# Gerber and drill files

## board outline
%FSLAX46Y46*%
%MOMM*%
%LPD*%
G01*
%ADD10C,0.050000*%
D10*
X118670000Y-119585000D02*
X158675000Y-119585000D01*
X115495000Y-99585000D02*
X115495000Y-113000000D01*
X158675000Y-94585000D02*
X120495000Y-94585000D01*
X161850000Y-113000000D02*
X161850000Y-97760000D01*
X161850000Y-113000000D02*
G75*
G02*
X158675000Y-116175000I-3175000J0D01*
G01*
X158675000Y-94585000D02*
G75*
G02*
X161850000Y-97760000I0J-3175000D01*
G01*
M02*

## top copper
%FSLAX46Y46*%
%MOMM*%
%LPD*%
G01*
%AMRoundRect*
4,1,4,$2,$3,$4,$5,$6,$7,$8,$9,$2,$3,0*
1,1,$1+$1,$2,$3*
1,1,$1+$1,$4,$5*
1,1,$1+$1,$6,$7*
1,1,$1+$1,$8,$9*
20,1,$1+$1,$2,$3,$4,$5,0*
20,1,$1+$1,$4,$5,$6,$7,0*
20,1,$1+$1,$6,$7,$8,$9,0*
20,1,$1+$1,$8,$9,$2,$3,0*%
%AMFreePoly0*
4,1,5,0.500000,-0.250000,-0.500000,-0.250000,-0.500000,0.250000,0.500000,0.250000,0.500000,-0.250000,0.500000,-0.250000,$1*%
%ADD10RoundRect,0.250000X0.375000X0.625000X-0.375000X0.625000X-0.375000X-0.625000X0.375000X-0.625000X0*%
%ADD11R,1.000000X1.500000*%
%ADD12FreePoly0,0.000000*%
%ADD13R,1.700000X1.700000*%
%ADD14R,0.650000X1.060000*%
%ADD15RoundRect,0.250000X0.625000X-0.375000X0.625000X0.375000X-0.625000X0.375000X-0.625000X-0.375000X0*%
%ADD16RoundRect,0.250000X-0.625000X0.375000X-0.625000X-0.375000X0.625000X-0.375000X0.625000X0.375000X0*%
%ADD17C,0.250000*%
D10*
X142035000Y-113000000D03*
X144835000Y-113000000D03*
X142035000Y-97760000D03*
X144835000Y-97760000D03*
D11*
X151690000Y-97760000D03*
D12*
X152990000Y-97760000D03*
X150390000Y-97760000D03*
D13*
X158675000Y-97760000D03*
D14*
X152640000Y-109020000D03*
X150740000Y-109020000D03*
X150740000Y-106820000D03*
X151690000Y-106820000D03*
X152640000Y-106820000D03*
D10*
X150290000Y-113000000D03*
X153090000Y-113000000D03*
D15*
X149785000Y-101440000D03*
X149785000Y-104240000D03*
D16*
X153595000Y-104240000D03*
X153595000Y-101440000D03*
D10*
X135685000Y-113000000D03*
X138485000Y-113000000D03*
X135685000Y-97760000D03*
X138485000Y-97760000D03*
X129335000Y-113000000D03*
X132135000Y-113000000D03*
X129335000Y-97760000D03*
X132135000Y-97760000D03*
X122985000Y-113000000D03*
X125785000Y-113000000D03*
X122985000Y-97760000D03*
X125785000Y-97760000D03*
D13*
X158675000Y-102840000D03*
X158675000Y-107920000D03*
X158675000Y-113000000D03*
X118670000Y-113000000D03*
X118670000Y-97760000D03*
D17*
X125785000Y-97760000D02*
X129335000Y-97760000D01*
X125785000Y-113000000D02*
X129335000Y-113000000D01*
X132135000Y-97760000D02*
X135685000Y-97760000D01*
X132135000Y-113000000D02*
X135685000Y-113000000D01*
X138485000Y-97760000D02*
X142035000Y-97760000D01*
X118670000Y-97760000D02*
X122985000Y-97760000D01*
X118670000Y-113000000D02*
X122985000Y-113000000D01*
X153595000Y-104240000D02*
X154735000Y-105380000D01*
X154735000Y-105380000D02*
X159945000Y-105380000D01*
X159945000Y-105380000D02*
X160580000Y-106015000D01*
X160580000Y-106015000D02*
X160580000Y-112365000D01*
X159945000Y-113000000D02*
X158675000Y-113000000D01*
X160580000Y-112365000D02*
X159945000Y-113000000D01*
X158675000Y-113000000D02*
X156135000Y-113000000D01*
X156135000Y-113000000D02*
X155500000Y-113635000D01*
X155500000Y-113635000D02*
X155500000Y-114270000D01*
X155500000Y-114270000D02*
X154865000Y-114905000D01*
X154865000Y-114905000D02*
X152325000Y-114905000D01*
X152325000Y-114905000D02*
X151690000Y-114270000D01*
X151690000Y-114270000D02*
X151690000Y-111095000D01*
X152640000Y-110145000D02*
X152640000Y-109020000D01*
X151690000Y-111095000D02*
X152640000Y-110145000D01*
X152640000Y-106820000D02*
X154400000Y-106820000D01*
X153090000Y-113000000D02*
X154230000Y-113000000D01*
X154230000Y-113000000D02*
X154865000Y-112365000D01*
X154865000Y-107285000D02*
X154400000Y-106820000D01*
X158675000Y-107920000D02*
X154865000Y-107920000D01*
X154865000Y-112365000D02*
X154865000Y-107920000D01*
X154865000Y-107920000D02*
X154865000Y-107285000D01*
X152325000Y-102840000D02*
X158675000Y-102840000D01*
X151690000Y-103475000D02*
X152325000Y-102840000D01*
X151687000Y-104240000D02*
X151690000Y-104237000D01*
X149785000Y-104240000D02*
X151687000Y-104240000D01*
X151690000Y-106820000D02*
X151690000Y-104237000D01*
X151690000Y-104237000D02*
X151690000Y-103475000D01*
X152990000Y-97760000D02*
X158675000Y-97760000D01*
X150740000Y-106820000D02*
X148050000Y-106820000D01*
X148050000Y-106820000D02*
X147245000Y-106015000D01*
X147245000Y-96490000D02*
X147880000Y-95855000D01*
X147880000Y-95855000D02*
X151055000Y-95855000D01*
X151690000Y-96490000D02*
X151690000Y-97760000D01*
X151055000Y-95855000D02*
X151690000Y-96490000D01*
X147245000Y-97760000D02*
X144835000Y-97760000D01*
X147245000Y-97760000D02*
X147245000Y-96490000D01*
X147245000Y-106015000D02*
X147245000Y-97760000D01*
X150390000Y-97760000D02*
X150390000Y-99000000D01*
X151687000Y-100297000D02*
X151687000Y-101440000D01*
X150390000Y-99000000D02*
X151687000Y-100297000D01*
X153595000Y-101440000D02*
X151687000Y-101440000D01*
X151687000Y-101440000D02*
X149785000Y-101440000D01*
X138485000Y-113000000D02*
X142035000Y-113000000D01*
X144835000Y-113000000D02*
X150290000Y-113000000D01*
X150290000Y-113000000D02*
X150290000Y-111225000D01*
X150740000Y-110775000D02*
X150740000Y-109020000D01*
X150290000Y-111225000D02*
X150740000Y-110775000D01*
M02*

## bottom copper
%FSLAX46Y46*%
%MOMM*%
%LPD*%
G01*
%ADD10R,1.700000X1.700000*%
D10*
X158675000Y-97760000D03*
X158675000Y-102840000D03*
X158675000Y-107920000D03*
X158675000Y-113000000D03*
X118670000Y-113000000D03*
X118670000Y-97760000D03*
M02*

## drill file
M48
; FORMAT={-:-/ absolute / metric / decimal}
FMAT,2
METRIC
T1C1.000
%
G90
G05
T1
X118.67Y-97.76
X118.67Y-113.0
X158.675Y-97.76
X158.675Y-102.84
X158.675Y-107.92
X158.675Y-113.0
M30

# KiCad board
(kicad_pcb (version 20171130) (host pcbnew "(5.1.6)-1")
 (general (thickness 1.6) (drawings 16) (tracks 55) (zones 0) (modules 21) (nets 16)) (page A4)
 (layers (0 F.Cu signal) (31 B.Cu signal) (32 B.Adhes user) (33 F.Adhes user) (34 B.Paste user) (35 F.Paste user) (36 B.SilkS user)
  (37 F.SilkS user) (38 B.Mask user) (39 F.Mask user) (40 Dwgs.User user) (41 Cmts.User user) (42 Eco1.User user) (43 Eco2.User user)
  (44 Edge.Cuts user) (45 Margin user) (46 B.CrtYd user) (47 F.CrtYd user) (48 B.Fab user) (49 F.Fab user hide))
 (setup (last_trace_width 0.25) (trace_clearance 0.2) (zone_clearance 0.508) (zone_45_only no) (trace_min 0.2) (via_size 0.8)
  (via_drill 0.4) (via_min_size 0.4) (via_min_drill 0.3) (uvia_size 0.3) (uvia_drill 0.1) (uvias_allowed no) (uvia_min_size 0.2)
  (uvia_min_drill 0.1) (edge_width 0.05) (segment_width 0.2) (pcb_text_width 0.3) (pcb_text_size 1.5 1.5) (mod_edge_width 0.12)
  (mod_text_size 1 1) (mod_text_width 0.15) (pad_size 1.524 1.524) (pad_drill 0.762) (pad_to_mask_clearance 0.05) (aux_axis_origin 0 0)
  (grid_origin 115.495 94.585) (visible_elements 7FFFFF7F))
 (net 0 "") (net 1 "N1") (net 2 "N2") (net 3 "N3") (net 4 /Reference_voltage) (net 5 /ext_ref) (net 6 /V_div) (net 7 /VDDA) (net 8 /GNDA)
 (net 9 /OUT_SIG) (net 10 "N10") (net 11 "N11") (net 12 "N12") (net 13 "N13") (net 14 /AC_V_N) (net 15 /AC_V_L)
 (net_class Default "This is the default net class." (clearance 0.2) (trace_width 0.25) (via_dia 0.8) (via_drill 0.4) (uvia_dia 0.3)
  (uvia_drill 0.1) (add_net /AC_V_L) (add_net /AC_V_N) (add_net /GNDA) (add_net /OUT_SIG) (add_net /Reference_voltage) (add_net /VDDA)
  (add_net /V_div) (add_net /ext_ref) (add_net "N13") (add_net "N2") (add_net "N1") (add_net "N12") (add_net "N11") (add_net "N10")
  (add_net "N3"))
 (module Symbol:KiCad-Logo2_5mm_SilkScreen (layer F.Cu) (at 129.465 105.38)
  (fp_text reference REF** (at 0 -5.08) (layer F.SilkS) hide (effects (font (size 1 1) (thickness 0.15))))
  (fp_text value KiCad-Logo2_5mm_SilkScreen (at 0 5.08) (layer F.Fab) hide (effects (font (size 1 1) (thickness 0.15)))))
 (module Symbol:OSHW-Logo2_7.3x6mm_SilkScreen (layer F.Cu) (at 142.165 105.38)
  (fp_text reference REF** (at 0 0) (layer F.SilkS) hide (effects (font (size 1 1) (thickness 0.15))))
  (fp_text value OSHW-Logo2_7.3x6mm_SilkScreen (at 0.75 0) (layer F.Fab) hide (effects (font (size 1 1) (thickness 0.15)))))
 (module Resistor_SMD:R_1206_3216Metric (layer F.Cu) (at 143.435 113 180)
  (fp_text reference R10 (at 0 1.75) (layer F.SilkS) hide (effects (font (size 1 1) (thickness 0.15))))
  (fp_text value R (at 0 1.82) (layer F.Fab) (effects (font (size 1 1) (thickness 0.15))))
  (pad 2 smd roundrect (at 1.4 0 180) (size 1.25 1.75) (layers F.Cu F.Paste F.Mask) (roundrect_rratio 0.2) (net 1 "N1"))
  (pad 1 smd roundrect (at -1.4 0 180) (size 1.25 1.75) (layers F.Cu F.Paste F.Mask) (roundrect_rratio 0.2) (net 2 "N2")))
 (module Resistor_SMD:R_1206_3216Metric (layer F.Cu) (at 143.435 97.76 180)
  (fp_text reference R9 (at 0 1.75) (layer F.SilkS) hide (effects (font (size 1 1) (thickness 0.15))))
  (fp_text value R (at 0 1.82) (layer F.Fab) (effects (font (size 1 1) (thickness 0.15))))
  (pad 2 smd roundrect (at 1.4 0 180) (size 1.25 1.75) (layers F.Cu F.Paste F.Mask) (roundrect_rratio 0.2) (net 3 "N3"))
  (pad 1 smd roundrect (at -1.4 0 180) (size 1.25 1.75) (layers F.Cu F.Paste F.Mask) (roundrect_rratio 0.2) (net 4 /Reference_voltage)))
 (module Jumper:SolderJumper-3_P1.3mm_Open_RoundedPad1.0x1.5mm (layer F.Cu) (at 151.69 97.76)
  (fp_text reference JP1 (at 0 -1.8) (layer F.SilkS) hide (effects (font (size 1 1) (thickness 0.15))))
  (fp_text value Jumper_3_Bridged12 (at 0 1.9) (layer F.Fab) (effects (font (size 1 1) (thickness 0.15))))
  (pad 2 smd rect (at 0 0) (size 1 1.5) (layers F.Cu F.Mask) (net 4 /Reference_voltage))
  (pad 3 smd custom (at 1.3 0) (size 1 0.5) (layers F.Cu F.Mask) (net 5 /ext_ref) (zone_connect 2)
   (options (clearance outline) (anchor rect)) (primitives))
  (pad 1 smd custom (at -1.3 0) (size 1 0.5) (layers F.Cu F.Mask) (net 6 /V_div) (zone_connect 2)
   (options (clearance outline) (anchor rect)) (primitives)))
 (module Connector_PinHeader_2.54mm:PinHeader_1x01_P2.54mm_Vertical (layer F.Cu) (at 158.675 97.76)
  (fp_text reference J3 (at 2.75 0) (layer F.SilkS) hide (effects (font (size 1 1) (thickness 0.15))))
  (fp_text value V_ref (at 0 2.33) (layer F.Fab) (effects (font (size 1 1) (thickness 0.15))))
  (pad 1 thru_hole rect (at 0 0) (size 1.7 1.7) (drill 1) (layers *.Cu *.Mask) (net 5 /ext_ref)))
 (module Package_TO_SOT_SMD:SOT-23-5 (layer F.Cu) (at 151.69 107.92 270)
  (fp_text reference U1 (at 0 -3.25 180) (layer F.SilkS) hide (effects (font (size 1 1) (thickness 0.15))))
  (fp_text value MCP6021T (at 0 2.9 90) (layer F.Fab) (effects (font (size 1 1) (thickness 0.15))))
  (pad 5 smd rect (at 1.1 -0.95 270) (size 1.06 0.65) (layers F.Cu F.Paste F.Mask) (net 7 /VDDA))
  (pad 4 smd rect (at 1.1 0.95 270) (size 1.06 0.65) (layers F.Cu F.Paste F.Mask) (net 2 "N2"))
  (pad 3 smd rect (at -1.1 0.95 270) (size 1.06 0.65) (layers F.Cu F.Paste F.Mask) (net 4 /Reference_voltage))
  (pad 2 smd rect (at -1.1 0 270) (size 1.06 0.65) (layers F.Cu F.Paste F.Mask) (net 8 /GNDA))
  (pad 1 smd rect (at -1.1 -0.95 270) (size 1.06 0.65) (layers F.Cu F.Paste F.Mask) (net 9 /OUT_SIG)))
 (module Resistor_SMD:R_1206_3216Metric (layer F.Cu) (at 151.69 113 180)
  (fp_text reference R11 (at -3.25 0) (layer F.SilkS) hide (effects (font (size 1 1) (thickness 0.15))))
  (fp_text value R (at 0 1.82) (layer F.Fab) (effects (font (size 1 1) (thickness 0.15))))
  (pad 2 smd roundrect (at 1.4 0 180) (size 1.25 1.75) (layers F.Cu F.Paste F.Mask) (roundrect_rratio 0.2) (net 2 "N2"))
  (pad 1 smd roundrect (at -1.4 0 180) (size 1.25 1.75) (layers F.Cu F.Paste F.Mask) (roundrect_rratio 0.2) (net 9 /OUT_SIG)))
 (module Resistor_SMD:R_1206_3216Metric (layer F.Cu) (at 149.785 102.84 90)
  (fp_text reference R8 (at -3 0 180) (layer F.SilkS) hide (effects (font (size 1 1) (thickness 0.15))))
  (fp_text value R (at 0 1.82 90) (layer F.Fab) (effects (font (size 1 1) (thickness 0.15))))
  (pad 2 smd roundrect (at 1.4 0 90) (size 1.25 1.75) (layers F.Cu F.Paste F.Mask) (roundrect_rratio 0.2) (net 6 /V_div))
  (pad 1 smd roundrect (at -1.4 0 90) (size 1.25 1.75) (layers F.Cu F.Paste F.Mask) (roundrect_rratio 0.2) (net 8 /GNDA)))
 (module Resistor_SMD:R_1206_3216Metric (layer F.Cu) (at 153.595 102.84 270)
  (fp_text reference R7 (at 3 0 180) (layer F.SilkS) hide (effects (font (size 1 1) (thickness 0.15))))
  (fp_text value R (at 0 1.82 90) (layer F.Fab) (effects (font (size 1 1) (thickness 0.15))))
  (pad 2 smd roundrect (at 1.4 0 270) (size 1.25 1.75) (layers F.Cu F.Paste F.Mask) (roundrect_rratio 0.2) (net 7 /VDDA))
  (pad 1 smd roundrect (at -1.4 0 270) (size 1.25 1.75) (layers F.Cu F.Paste F.Mask) (roundrect_rratio 0.2) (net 6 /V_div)))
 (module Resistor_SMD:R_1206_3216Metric (layer F.Cu) (at 137.085 113 180)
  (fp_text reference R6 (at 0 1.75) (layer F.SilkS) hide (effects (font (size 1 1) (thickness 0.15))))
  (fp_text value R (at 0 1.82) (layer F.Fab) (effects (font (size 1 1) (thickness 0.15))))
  (pad 2 smd roundrect (at 1.4 0 180) (size 1.25 1.75) (layers F.Cu F.Paste F.Mask) (roundrect_rratio 0.2) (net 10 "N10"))
  (pad 1 smd roundrect (at -1.4 0 180) (size 1.25 1.75) (layers F.Cu F.Paste F.Mask) (roundrect_rratio 0.2) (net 1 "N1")))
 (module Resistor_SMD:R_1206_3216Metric (layer F.Cu) (at 137.085 97.76 180)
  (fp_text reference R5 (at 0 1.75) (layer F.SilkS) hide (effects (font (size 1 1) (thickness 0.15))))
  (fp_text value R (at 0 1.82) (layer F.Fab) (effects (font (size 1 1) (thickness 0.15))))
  (pad 2 smd roundrect (at 1.4 0 180) (size 1.25 1.75) (layers F.Cu F.Paste F.Mask) (roundrect_rratio 0.2) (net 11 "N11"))
  (pad 1 smd roundrect (at -1.4 0 180) (size 1.25 1.75) (layers F.Cu F.Paste F.Mask) (roundrect_rratio 0.2) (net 3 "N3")))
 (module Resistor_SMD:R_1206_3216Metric (layer F.Cu) (at 130.735 113 180)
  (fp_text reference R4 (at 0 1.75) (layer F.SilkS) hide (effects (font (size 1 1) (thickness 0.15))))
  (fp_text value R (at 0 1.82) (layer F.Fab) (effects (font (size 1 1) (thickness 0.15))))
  (pad 2 smd roundrect (at 1.4 0 180) (size 1.25 1.75) (layers F.Cu F.Paste F.Mask) (roundrect_rratio 0.2) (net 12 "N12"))
  (pad 1 smd roundrect (at -1.4 0 180) (size 1.25 1.75) (layers F.Cu F.Paste F.Mask) (roundrect_rratio 0.2) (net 10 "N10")))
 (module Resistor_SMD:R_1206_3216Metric (layer F.Cu) (at 130.735 97.76 180)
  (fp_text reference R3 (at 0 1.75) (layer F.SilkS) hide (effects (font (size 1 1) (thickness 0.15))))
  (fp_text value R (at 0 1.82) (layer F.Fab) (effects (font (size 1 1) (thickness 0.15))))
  (pad 2 smd roundrect (at 1.4 0 180) (size 1.25 1.75) (layers F.Cu F.Paste F.Mask) (roundrect_rratio 0.2) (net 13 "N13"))
  (pad 1 smd roundrect (at -1.4 0 180) (size 1.25 1.75) (layers F.Cu F.Paste F.Mask) (roundrect_rratio 0.2) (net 11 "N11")))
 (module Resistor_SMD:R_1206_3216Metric (layer F.Cu) (at 124.385 113 180)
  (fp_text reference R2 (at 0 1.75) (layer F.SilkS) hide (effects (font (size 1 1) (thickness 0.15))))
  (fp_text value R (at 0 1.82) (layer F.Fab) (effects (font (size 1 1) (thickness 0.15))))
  (pad 2 smd roundrect (at 1.4 0 180) (size 1.25 1.75) (layers F.Cu F.Paste F.Mask) (roundrect_rratio 0.2) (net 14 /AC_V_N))
  (pad 1 smd roundrect (at -1.4 0 180) (size 1.25 1.75) (layers F.Cu F.Paste F.Mask) (roundrect_rratio 0.2) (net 12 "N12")))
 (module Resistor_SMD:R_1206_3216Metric (layer F.Cu) (at 124.385 97.76 180)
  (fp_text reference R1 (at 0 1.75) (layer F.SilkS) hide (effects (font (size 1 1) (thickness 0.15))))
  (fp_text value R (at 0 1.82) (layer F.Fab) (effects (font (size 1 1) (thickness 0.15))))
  (pad 2 smd roundrect (at 1.4 0 180) (size 1.25 1.75) (layers F.Cu F.Paste F.Mask) (roundrect_rratio 0.2) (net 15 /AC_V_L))
  (pad 1 smd roundrect (at -1.4 0 180) (size 1.25 1.75) (layers F.Cu F.Paste F.Mask) (roundrect_rratio 0.2) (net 13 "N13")))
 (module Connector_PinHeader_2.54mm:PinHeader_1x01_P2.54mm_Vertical (layer F.Cu) (at 158.675 102.84)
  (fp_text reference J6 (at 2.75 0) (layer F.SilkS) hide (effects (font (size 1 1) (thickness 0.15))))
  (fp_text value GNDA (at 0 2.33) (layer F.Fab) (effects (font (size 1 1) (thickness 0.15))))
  (pad 1 thru_hole rect (at 0 0) (size 1.7 1.7) (drill 1) (layers *.Cu *.Mask) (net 8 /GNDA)))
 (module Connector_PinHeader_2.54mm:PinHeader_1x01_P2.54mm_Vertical (layer F.Cu) (at 158.675 107.92)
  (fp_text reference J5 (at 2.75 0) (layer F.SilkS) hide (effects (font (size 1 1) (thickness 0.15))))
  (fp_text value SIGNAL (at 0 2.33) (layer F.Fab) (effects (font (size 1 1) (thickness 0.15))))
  (pad 1 thru_hole rect (at 0 0) (size 1.7 1.7) (drill 1) (layers *.Cu *.Mask) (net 9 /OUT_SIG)))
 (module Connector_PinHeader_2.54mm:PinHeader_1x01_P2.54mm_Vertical (layer F.Cu) (at 158.675 113)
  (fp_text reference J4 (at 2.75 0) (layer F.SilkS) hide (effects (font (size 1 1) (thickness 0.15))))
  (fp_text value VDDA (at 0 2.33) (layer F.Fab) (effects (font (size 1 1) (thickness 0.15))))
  (pad 1 thru_hole rect (at 0 0) (size 1.7 1.7) (drill 1) (layers *.Cu *.Mask) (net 7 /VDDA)))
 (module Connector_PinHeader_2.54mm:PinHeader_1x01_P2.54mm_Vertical (layer F.Cu) (at 118.67 113)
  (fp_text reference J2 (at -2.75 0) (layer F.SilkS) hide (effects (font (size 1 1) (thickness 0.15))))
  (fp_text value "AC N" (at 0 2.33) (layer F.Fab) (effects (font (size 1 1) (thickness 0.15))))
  (pad 1 thru_hole rect (at 0 0) (size 1.7 1.7) (drill 1) (layers *.Cu *.Mask) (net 14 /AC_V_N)))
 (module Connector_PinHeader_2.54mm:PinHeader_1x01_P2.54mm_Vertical (layer F.Cu) (at 118.67 97.76)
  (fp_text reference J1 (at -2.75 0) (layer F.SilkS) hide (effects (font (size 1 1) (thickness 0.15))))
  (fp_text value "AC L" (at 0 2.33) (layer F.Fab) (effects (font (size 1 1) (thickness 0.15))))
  (pad 1 thru_hole rect (at 0 0) (size 1.7 1.7) (drill 1) (layers *.Cu *.Mask) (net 15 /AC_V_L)))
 (gr_line (start 118.67 119.585) (end 158.675 119.585) (layer Edge.Cuts) (width 0.05))
 (gr_line (start 115.495 99.585) (end 115.495 113) (layer Edge.Cuts) (width 0.05))
 (gr_line (start 158.675 94.585) (end 120.495 94.585) (layer Edge.Cuts) (width 0.05))
 (gr_line (start 161.85 113) (end 161.85 97.76) (layer Edge.Cuts) (width 0.05))
 (gr_arc (start 158.675 113) (end 158.675 116.175) (angle -90) (layer Edge.Cuts) (width 0.05))
 (gr_arc (start 158.675 97.76) (end 161.85 97.76) (angle -90) (layer Edge.Cuts) (width 0.05))
 (segment (start 125.785 97.76) (end 129.335 97.76) (width 0.25) (layer F.Cu) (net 13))
 (segment (start 125.785 113) (end 129.335 113) (width 0.25) (layer F.Cu) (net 12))
 (segment (start 132.135 97.76) (end 135.685 97.76) (width 0.25) (layer F.Cu) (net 11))
 (segment (start 132.135 113) (end 135.685 113) (width 0.25) (layer F.Cu) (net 10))
 (segment (start 138.485 97.76) (end 142.035 97.76) (width 0.25) (layer F.Cu) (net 3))
 (segment (start 118.67 97.76) (end 122.985 97.76) (width 0.25) (layer F.Cu) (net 15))
 (segment (start 118.67 113) (end 122.985 113) (width 0.25) (layer F.Cu) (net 14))
 (segment (start 153.595 104.24) (end 154.735 105.38) (width 0.25) (layer F.Cu) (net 7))
 (segment (start 154.735 105.38) (end 159.945 105.38) (width 0.25) (layer F.Cu) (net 7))
 (segment (start 159.945 105.38) (end 160.58 106.015) (width 0.25) (layer F.Cu) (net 7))
 (segment (start 160.58 106.015) (end 160.58 112.365) (width 0.25) (layer F.Cu) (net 7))
 (segment (start 159.945 113) (end 158.675 113) (width 0.25) (layer F.Cu) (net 7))
 (segment (start 160.58 112.365) (end 159.945 113) (width 0.25) (layer F.Cu) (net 7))
 (segment (start 158.675 113) (end 156.135 113) (width 0.25) (layer F.Cu) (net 7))
 (segment (start 156.135 113) (end 155.5 113.635) (width 0.25) (layer F.Cu) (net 7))
 (segment (start 155.5 113.635) (end 155.5 114.27) (width 0.25) (layer F.Cu) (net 7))
 (segment (start 155.5 114.27) (end 154.865 114.905) (width 0.25) (layer F.Cu) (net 7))
 (segment (start 154.865 114.905) (end 152.325 114.905) (width 0.25) (layer F.Cu) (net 7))
 (segment (start 152.325 114.905) (end 151.69 114.27) (width 0.25) (layer F.Cu) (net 7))
 (segment (start 151.69 114.27) (end 151.69 111.095) (width 0.25) (layer F.Cu) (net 7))
 (segment (start 152.64 110.145) (end 152.64 109.02) (width 0.25) (layer F.Cu) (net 7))
 (segment (start 151.69 111.095) (end 152.64 110.145) (width 0.25) (layer F.Cu) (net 7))
 (segment (start 152.64 106.82) (end 154.4 106.82) (width 0.25) (layer F.Cu) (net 9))
 (segment (start 153.09 113) (end 154.23 113) (width 0.25) (layer F.Cu) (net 9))
 (segment (start 154.23 113) (end 154.865 112.365) (width 0.25) (layer F.Cu) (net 9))
 (segment (start 154.865 107.285) (end 154.4 106.82) (width 0.25) (layer F.Cu) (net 9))
 (segment (start 158.675 107.92) (end 154.865 107.92) (width 0.25) (layer F.Cu) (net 9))
 (segment (start 154.865 112.365) (end 154.865 107.92) (width 0.25) (layer F.Cu) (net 9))
 (segment (start 154.865 107.92) (end 154.865 107.285) (width 0.25) (layer F.Cu) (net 9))
 (segment (start 152.325 102.84) (end 158.675 102.84) (width 0.25) (layer F.Cu) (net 8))
 (segment (start 151.69 103.475) (end 152.325 102.84) (width 0.25) (layer F.Cu) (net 8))
 (segment (start 151.687 104.24) (end 151.69 104.237) (width 0.25) (layer F.Cu) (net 8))
 (segment (start 149.785 104.24) (end 151.687 104.24) (width 0.25) (layer F.Cu) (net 8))
 (segment (start 151.69 106.82) (end 151.69 104.237) (width 0.25) (layer F.Cu) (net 8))
 (segment (start 151.69 104.237) (end 151.69 103.475) (width 0.25) (layer F.Cu) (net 8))
 (segment (start 152.99 97.76) (end 158.675 97.76) (width 0.25) (layer F.Cu) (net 5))
 (segment (start 150.74 106.82) (end 148.05 106.82) (width 0.25) (layer F.Cu) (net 4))
 (segment (start 148.05 106.82) (end 147.245 106.015) (width 0.25) (layer F.Cu) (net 4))
 (segment (start 147.245 96.49) (end 147.88 95.855) (width 0.25) (layer F.Cu) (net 4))
 (segment (start 147.88 95.855) (end 151.055 95.855) (width 0.25) (layer F.Cu) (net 4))
 (segment (start 151.69 96.49) (end 151.69 97.76) (width 0.25) (layer F.Cu) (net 4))
 (segment (start 151.055 95.855) (end 151.69 96.49) (width 0.25) (layer F.Cu) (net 4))
 (segment (start 147.245 97.76) (end 144.835 97.76) (width 0.25) (layer F.Cu) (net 4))
 (segment (start 147.245 97.76) (end 147.245 96.49) (width 0.25) (layer F.Cu) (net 4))
 (segment (start 147.245 106.015) (end 147.245 97.76) (width 0.25) (layer F.Cu) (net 4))
 (segment (start 150.39 97.76) (end 150.39 99) (width 0.25) (layer F.Cu) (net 6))
 (segment (start 151.687 100.297) (end 151.687 101.44) (width 0.25) (layer F.Cu) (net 6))
 (segment (start 150.39 99) (end 151.687 100.297) (width 0.25) (layer F.Cu) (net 6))
 (segment (start 153.595 101.44) (end 151.687 101.44) (width 0.25) (layer F.Cu) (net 6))
 (segment (start 151.687 101.44) (end 149.785 101.44) (width 0.25) (layer F.Cu) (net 6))
 (segment (start 138.485 113) (end 142.035 113) (width 0.25) (layer F.Cu) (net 1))
 (segment (start 144.835 113) (end 150.29 113) (width 0.25) (layer F.Cu) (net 2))
 (segment (start 150.29 113) (end 150.29 111.225) (width 0.25) (layer F.Cu) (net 2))
 (segment (start 150.74 110.775) (end 150.74 109.02) (width 0.25) (layer F.Cu) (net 2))
 (segment (start 150.29 111.225) (end 150.74 110.775) (width 0.25) (layer F.Cu) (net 2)))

